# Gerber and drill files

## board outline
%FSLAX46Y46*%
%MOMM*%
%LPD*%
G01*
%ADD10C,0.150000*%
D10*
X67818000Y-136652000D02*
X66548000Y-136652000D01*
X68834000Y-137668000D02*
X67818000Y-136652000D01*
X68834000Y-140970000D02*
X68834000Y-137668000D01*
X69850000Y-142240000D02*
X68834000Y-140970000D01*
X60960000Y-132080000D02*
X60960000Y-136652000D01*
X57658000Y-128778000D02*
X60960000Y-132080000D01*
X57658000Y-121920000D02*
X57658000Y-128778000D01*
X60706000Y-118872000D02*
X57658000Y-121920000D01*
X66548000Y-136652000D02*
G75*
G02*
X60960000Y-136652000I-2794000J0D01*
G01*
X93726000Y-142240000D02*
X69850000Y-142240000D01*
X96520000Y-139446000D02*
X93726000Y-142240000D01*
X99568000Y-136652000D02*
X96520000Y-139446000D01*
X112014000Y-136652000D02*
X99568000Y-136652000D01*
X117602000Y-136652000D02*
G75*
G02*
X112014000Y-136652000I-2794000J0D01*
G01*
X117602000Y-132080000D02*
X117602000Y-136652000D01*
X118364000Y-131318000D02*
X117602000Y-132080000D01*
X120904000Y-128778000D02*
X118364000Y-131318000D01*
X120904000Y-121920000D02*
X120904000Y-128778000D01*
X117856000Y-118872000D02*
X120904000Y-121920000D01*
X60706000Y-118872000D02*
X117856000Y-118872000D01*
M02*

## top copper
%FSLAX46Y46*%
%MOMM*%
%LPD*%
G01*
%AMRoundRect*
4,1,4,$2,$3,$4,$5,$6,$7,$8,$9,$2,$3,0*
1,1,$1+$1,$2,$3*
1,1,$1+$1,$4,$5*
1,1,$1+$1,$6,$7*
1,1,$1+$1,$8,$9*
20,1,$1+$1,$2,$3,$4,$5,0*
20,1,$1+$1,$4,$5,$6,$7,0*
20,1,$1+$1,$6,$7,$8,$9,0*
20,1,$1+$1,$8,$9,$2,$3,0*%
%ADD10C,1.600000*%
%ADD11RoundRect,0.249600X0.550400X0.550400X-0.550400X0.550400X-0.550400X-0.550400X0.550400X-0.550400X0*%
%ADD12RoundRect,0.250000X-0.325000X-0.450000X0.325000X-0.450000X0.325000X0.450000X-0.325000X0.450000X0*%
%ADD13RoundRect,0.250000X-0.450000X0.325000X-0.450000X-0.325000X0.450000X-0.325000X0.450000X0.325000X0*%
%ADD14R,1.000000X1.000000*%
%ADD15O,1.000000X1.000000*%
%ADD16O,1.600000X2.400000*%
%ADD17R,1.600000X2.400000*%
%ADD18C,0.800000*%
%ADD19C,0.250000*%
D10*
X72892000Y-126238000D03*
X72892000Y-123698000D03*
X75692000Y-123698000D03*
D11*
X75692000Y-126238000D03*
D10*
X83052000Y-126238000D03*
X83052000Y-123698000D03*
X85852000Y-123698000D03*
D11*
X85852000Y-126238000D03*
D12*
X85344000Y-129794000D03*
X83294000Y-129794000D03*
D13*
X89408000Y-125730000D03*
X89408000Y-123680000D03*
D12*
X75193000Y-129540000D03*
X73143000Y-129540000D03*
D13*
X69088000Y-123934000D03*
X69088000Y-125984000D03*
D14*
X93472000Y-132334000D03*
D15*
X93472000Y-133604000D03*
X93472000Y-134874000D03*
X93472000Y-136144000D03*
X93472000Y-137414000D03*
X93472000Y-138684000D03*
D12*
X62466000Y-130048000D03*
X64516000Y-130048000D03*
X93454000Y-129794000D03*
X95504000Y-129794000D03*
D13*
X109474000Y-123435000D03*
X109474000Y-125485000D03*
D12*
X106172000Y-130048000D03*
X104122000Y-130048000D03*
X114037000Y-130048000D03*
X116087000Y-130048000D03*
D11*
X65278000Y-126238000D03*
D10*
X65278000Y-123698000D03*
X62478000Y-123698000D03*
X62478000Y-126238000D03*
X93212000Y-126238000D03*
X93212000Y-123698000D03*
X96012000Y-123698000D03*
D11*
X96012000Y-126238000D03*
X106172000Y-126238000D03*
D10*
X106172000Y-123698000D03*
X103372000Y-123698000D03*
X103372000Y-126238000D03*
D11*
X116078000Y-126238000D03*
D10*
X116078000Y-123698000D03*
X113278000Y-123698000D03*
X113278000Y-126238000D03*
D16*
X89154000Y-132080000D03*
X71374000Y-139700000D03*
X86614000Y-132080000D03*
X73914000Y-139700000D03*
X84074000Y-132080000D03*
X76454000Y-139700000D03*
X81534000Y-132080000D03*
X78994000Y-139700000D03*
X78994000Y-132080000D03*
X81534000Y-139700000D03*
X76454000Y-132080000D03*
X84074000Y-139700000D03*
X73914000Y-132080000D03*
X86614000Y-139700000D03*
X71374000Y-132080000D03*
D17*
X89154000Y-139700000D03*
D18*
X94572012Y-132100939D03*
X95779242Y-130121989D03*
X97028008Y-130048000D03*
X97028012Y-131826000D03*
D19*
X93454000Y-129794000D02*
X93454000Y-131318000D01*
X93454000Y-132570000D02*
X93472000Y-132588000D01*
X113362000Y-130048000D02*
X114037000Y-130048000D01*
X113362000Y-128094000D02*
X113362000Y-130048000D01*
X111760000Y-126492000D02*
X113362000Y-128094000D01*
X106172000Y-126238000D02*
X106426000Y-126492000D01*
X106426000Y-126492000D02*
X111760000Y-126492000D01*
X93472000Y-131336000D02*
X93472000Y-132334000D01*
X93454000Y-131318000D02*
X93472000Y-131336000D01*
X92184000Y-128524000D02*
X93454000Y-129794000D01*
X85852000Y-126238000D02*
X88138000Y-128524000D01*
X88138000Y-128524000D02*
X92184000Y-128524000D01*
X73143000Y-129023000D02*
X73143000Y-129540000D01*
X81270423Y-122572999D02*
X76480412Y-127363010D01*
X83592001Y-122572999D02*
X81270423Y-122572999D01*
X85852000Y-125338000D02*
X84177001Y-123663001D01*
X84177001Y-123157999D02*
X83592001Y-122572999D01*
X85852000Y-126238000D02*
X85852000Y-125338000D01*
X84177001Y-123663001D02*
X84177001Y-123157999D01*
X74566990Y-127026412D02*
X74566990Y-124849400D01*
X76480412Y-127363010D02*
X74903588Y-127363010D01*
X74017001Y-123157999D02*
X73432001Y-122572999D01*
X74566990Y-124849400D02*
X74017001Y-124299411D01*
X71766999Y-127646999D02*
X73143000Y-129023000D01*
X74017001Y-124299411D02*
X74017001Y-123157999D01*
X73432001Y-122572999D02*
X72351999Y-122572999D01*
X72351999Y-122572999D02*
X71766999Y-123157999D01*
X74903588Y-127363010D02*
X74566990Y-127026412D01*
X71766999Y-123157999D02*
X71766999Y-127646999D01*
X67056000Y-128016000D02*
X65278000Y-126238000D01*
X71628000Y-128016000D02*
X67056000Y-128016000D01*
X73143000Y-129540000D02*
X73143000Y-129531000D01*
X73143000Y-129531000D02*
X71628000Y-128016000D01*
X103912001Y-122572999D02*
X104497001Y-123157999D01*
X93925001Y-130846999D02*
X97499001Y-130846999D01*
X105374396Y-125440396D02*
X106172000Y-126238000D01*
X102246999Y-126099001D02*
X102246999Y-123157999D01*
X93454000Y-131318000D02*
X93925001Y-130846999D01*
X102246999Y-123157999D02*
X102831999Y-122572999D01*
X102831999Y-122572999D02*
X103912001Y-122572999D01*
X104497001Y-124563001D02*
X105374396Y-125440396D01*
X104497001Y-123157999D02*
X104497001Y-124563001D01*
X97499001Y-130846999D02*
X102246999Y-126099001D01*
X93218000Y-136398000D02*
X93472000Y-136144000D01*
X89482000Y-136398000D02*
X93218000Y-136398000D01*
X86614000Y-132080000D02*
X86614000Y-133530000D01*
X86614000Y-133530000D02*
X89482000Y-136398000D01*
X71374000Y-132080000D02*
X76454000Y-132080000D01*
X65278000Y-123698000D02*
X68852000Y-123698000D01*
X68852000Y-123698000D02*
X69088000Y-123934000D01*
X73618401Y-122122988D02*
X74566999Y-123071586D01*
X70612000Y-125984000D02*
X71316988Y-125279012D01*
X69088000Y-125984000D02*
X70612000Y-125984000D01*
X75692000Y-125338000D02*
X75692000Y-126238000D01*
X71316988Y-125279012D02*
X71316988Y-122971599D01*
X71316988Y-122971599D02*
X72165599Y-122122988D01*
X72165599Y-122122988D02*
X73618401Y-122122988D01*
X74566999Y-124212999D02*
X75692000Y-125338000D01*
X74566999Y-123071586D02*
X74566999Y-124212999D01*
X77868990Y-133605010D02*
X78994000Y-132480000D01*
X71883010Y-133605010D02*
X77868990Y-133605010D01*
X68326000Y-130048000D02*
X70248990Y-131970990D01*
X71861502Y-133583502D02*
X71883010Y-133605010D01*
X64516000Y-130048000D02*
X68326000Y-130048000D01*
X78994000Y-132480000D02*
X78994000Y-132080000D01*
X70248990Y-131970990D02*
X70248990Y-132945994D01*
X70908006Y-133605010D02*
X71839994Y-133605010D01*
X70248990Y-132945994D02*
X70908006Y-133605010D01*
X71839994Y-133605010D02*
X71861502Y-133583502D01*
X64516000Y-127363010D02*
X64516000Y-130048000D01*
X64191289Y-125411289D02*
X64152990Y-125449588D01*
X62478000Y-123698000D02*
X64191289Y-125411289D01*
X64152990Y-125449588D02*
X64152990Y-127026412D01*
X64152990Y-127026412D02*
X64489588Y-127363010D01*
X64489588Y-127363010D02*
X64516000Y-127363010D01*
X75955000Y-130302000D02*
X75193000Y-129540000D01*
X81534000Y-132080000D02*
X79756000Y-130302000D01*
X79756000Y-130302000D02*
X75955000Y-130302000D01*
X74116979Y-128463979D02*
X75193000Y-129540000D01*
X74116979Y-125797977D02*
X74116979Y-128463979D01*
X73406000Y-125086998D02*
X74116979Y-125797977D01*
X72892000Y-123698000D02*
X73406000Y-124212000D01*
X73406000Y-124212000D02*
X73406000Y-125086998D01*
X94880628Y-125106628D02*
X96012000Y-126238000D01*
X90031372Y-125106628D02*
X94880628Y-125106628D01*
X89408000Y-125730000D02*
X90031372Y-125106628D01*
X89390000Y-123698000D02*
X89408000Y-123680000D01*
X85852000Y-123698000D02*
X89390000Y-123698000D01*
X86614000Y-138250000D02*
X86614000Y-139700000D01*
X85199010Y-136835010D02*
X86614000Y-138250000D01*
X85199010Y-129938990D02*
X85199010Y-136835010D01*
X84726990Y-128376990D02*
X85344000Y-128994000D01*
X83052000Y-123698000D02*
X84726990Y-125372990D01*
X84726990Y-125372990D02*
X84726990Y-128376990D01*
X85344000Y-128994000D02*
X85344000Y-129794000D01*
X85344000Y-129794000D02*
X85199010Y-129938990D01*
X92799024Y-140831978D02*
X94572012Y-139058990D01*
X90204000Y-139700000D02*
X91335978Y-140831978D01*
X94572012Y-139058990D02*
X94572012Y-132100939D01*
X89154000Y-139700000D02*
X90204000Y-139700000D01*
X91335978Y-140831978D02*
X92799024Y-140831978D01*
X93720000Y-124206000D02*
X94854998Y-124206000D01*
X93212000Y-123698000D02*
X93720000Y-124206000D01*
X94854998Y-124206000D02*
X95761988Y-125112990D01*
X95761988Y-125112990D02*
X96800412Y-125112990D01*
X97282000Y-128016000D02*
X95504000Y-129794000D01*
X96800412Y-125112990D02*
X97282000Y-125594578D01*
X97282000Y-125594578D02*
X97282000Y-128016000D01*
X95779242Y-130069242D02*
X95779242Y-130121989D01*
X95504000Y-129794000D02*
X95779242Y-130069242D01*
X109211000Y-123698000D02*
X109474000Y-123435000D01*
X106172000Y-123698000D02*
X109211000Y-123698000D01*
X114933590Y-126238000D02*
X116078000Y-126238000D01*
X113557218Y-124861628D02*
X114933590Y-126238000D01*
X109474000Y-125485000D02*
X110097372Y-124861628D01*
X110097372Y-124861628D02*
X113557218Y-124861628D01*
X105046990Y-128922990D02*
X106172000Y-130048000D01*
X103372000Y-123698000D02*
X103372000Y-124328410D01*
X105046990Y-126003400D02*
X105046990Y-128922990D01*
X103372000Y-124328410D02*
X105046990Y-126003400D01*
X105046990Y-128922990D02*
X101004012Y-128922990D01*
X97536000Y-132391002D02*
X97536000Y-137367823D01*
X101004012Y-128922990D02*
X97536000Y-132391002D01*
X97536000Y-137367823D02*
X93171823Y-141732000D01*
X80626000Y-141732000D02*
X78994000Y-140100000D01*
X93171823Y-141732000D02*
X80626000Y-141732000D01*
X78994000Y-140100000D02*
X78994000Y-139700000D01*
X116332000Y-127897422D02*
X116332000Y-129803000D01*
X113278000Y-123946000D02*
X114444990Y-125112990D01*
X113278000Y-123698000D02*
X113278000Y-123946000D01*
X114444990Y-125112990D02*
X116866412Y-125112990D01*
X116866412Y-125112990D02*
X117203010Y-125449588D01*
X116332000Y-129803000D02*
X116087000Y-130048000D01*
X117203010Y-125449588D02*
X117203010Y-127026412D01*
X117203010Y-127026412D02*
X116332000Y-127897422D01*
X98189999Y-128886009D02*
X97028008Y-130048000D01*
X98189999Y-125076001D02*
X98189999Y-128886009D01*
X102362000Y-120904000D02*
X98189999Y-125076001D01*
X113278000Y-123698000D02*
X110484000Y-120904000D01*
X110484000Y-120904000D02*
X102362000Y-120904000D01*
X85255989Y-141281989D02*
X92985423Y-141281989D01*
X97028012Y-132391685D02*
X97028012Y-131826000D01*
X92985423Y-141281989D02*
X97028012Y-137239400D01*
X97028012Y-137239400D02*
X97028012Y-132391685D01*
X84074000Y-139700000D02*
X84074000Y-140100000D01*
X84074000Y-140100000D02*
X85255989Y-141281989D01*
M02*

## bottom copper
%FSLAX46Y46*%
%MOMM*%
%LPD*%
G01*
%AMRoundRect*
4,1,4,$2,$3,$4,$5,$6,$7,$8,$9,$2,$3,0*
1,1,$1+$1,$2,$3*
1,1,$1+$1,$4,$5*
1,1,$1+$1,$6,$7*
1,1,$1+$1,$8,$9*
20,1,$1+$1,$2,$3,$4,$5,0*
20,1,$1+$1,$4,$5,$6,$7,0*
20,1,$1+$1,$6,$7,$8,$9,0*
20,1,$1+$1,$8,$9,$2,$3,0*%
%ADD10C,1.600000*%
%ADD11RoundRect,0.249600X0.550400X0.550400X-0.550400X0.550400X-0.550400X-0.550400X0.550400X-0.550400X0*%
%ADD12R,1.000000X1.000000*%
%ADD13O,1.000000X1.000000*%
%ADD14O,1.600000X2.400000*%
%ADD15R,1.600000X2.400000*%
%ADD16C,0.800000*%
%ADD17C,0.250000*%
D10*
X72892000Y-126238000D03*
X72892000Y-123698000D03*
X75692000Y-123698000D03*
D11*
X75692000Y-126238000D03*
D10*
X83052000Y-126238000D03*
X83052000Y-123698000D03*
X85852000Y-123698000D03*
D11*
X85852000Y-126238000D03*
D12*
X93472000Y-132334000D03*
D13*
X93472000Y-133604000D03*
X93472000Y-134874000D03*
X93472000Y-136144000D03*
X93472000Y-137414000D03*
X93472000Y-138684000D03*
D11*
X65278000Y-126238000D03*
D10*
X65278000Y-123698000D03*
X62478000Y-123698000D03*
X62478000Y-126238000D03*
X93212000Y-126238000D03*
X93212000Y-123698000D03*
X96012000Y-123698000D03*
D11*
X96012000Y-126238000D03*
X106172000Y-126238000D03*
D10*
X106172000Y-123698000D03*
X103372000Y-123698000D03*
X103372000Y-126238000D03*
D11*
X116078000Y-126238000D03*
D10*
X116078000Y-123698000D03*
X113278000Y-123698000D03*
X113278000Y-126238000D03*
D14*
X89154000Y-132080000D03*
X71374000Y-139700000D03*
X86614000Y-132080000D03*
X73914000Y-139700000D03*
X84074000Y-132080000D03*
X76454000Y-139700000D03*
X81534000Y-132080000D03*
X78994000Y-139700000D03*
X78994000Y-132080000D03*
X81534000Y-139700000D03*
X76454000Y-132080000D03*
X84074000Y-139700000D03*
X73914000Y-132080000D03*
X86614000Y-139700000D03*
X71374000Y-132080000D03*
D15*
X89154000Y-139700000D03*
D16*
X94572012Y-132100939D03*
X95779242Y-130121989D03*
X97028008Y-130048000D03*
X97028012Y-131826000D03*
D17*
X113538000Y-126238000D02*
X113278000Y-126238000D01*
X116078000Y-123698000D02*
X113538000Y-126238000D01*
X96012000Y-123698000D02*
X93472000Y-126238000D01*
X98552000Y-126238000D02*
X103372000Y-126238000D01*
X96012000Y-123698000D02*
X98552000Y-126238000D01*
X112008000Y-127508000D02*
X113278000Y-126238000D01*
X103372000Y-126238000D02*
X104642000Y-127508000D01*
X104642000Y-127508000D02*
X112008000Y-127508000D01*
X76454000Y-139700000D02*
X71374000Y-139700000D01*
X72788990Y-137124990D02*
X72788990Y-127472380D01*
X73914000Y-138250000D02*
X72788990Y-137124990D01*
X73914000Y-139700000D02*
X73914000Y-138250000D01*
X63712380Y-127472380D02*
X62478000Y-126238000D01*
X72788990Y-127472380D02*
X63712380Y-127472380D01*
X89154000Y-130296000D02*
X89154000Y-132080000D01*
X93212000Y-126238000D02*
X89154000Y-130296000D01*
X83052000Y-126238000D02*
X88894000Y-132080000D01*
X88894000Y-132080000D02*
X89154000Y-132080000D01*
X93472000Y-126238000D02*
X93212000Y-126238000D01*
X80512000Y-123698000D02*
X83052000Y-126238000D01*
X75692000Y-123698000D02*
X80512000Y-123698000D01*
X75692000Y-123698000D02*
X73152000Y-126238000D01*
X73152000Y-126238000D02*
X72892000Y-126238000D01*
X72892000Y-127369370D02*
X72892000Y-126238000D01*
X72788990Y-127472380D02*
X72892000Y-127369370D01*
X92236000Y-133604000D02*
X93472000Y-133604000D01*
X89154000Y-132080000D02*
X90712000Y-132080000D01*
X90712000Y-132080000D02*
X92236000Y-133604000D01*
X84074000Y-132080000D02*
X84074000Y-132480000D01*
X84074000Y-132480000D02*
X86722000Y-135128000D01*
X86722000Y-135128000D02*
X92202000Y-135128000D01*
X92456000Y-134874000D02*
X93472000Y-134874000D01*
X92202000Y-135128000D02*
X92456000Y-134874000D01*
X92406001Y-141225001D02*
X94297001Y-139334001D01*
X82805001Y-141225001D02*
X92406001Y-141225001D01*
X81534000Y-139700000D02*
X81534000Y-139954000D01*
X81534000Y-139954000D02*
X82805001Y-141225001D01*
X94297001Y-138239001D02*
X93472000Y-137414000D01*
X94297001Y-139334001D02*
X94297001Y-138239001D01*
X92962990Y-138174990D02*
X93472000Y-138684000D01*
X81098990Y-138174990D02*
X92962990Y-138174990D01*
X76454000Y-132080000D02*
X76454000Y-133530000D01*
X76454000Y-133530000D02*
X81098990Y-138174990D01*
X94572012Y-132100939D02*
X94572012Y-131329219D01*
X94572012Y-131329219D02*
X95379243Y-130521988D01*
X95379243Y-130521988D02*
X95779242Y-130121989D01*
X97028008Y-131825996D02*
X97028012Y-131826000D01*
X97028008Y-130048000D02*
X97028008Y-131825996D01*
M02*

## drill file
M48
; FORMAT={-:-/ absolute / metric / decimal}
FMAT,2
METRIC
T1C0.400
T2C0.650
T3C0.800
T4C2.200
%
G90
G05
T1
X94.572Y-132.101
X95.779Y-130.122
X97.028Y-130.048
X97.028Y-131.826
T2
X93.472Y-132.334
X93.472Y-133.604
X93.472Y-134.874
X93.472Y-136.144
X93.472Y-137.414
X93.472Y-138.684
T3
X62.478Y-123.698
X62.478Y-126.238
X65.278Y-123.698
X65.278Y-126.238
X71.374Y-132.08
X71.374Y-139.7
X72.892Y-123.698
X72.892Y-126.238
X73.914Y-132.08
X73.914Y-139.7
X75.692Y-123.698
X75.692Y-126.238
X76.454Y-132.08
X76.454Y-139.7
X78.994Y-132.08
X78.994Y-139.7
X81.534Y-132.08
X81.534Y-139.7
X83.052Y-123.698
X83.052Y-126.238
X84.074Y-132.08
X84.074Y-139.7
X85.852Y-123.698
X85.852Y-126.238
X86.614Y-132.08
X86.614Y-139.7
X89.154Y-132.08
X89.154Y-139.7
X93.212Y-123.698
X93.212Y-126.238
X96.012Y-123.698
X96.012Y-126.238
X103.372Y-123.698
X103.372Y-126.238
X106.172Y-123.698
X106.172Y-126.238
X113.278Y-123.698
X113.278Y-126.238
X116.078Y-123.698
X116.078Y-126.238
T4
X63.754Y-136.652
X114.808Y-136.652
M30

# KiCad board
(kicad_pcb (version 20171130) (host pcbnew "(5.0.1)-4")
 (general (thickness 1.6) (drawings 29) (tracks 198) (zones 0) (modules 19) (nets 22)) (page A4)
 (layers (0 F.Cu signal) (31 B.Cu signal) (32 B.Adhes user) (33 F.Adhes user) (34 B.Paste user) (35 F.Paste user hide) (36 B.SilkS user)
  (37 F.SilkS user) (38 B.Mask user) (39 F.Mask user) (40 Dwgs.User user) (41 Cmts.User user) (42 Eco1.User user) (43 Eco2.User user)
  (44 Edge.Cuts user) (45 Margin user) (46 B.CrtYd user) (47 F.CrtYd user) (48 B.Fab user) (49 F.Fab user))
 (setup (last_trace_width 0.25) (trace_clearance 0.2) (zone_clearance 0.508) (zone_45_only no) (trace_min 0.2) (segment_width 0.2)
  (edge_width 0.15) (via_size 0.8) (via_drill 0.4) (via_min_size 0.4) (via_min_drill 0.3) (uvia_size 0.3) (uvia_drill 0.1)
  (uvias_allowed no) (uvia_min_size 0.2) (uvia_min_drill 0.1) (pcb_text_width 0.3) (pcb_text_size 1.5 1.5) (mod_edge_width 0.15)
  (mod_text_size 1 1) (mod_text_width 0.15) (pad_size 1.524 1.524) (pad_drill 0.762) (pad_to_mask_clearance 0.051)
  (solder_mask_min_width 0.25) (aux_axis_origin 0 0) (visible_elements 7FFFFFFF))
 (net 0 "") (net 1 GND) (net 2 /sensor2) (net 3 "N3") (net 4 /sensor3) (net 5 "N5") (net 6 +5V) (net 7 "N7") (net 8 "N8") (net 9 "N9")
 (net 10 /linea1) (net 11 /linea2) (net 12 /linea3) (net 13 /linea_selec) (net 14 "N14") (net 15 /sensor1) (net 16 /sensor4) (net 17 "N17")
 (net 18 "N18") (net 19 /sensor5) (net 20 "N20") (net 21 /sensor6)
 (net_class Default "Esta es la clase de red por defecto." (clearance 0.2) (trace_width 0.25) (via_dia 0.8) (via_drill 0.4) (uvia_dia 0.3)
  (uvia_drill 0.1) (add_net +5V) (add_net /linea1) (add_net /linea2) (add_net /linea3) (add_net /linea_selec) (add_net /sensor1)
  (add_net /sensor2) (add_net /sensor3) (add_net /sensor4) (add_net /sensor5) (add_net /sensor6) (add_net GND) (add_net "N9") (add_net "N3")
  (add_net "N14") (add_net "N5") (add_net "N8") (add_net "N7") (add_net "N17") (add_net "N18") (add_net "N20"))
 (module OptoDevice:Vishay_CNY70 (layer F.Cu) (at 75.692 126.238 180)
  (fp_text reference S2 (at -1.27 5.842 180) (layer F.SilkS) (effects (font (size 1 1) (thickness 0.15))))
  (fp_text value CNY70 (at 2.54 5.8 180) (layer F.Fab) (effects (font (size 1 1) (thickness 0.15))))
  (pad 4 thru_hole circle (at 2.8 0 180) (size 1.6 1.6) (drill 0.8) (layers *.Cu *.Mask) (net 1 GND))
  (pad 3 thru_hole circle (at 2.8 2.54 180) (size 1.6 1.6) (drill 0.8) (layers *.Cu *.Mask) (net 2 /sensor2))
  (pad 2 thru_hole circle (at 0 2.54 180) (size 1.6 1.6) (drill 0.8) (layers *.Cu *.Mask) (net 1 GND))
  (pad 1 thru_hole roundrect (at 0 0 180) (size 1.6 1.6) (drill 0.8) (layers *.Cu *.Mask) (roundrect_rratio 0.156) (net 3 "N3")))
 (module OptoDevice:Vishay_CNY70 (layer F.Cu) (at 85.852 126.238 180)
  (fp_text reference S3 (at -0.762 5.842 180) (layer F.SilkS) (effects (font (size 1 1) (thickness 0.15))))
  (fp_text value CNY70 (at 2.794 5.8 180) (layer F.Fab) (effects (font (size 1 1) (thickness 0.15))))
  (pad 4 thru_hole circle (at 2.8 0 180) (size 1.6 1.6) (drill 0.8) (layers *.Cu *.Mask) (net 1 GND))
  (pad 3 thru_hole circle (at 2.8 2.54 180) (size 1.6 1.6) (drill 0.8) (layers *.Cu *.Mask) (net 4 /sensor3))
  (pad 2 thru_hole circle (at 0 2.54 180) (size 1.6 1.6) (drill 0.8) (layers *.Cu *.Mask) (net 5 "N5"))
  (pad 1 thru_hole roundrect (at 0 0 180) (size 1.6 1.6) (drill 0.8) (layers *.Cu *.Mask) (roundrect_rratio 0.156) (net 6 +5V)))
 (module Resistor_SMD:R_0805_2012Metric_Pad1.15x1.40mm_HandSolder (layer F.Cu) (at 84.319 129.794)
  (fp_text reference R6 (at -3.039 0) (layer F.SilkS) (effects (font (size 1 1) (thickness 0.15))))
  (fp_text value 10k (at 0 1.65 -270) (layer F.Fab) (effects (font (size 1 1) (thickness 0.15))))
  (pad 2 smd roundrect (at 1.025 0) (size 1.15 1.4) (layers F.Cu F.Paste F.Mask) (roundrect_rratio 0.217391) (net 4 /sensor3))
  (pad 1 smd roundrect (at -1.025 0) (size 1.15 1.4) (layers F.Cu F.Paste F.Mask) (roundrect_rratio 0.217391) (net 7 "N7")))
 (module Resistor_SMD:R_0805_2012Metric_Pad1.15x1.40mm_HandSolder (layer F.Cu) (at 89.408 124.705 270)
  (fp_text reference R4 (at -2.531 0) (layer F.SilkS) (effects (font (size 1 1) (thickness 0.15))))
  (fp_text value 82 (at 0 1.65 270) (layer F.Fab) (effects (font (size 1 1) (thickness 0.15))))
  (pad 2 smd roundrect (at 1.025 0 270) (size 1.15 1.4) (layers F.Cu F.Paste F.Mask) (roundrect_rratio 0.217391) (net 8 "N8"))
  (pad 1 smd roundrect (at -1.025 0 270) (size 1.15 1.4) (layers F.Cu F.Paste F.Mask) (roundrect_rratio 0.217391) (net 5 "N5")))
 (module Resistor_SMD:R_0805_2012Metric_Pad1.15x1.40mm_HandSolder (layer F.Cu) (at 74.168 129.54)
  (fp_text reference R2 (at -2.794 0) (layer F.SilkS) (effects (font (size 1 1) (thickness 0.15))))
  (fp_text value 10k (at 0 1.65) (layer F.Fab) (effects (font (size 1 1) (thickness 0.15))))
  (pad 2 smd roundrect (at 1.025 0) (size 1.15 1.4) (layers F.Cu F.Paste F.Mask) (roundrect_rratio 0.217391) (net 2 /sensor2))
  (pad 1 smd roundrect (at -1.025 0) (size 1.15 1.4) (layers F.Cu F.Paste F.Mask) (roundrect_rratio 0.217391) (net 6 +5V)))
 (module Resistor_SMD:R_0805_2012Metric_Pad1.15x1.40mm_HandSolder (layer F.Cu) (at 69.088 124.959 270)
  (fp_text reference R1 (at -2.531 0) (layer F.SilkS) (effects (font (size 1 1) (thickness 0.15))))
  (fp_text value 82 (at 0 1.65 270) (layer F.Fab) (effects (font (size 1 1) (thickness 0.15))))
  (pad 1 smd roundrect (at -1.025 0 270) (size 1.15 1.4) (layers F.Cu F.Paste F.Mask) (roundrect_rratio 0.217391) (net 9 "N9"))
  (pad 2 smd roundrect (at 1.025 0 270) (size 1.15 1.4) (layers F.Cu F.Paste F.Mask) (roundrect_rratio 0.217391) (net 3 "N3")))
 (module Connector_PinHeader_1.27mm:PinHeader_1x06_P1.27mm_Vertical (layer B.Cu) (at 93.472 132.334 180)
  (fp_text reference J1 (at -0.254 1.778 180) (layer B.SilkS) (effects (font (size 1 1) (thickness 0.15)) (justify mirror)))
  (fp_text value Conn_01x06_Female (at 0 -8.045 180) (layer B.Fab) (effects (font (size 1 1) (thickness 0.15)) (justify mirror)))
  (pad 1 thru_hole rect (at 0 0 180) (size 1 1) (drill 0.65) (layers *.Cu *.Mask) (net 6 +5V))
  (pad 2 thru_hole oval (at 0 -1.27 180) (size 1 1) (drill 0.65) (layers *.Cu *.Mask) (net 1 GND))
  (pad 3 thru_hole oval (at 0 -2.54 180) (size 1 1) (drill 0.65) (layers *.Cu *.Mask) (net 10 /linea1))
  (pad 4 thru_hole oval (at 0 -3.81 180) (size 1 1) (drill 0.65) (layers *.Cu *.Mask) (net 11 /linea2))
  (pad 5 thru_hole oval (at 0 -5.08 180) (size 1 1) (drill 0.65) (layers *.Cu *.Mask) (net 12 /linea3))
  (pad 6 thru_hole oval (at 0 -6.35 180) (size 1 1) (drill 0.65) (layers *.Cu *.Mask) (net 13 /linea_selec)))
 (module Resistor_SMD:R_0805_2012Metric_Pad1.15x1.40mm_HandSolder (layer F.Cu) (at 63.491 130.048)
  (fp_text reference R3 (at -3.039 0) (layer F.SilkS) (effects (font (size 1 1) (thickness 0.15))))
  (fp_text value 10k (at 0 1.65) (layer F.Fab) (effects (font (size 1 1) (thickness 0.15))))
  (pad 1 smd roundrect (at -1.025 0) (size 1.15 1.4) (layers F.Cu F.Paste F.Mask) (roundrect_rratio 0.217391) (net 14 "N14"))
  (pad 2 smd roundrect (at 1.025 0) (size 1.15 1.4) (layers F.Cu F.Paste F.Mask) (roundrect_rratio 0.217391) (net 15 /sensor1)))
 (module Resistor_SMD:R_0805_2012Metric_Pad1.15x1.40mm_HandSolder (layer F.Cu) (at 94.479 129.794)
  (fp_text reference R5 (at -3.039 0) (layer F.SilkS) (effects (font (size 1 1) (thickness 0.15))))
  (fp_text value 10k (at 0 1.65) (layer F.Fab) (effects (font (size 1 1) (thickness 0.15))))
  (pad 1 smd roundrect (at -1.025 0) (size 1.15 1.4) (layers F.Cu F.Paste F.Mask) (roundrect_rratio 0.217391) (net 6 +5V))
  (pad 2 smd roundrect (at 1.025 0) (size 1.15 1.4) (layers F.Cu F.Paste F.Mask) (roundrect_rratio 0.217391) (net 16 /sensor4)))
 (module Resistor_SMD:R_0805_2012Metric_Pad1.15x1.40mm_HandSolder (layer F.Cu) (at 109.474 124.46 270)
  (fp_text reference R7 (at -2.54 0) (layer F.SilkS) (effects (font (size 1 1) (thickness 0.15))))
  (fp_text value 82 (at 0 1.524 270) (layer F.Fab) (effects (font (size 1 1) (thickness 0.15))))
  (pad 1 smd roundrect (at -1.025 0 270) (size 1.15 1.4) (layers F.Cu F.Paste F.Mask) (roundrect_rratio 0.217391) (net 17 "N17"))
  (pad 2 smd roundrect (at 1.025 0 270) (size 1.15 1.4) (layers F.Cu F.Paste F.Mask) (roundrect_rratio 0.217391) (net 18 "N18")))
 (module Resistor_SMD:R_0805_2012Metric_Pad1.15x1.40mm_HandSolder (layer F.Cu) (at 105.147 130.048)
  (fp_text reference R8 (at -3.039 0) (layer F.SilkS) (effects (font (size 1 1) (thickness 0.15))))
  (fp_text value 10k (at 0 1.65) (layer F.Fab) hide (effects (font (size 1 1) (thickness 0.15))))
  (pad 2 smd roundrect (at 1.025 0) (size 1.15 1.4) (layers F.Cu F.Paste F.Mask) (roundrect_rratio 0.217391) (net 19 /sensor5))
  (pad 1 smd roundrect (at -1.025 0) (size 1.15 1.4) (layers F.Cu F.Paste F.Mask) (roundrect_rratio 0.217391) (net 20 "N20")))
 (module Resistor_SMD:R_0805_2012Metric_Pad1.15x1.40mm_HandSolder (layer F.Cu) (at 115.062 130.048)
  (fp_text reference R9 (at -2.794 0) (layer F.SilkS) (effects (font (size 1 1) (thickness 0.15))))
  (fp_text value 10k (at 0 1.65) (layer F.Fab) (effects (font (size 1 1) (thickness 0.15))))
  (pad 1 smd roundrect (at -1.025 0) (size 1.15 1.4) (layers F.Cu F.Paste F.Mask) (roundrect_rratio 0.217391) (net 6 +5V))
  (pad 2 smd roundrect (at 1.025 0) (size 1.15 1.4) (layers F.Cu F.Paste F.Mask) (roundrect_rratio 0.217391) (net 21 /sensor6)))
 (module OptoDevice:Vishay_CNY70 (layer F.Cu) (at 65.278 126.238 180)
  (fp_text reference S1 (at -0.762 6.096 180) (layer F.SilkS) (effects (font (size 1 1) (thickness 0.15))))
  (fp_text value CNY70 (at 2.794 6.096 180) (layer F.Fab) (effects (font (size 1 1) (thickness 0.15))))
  (pad 1 thru_hole roundrect (at 0 0 180) (size 1.6 1.6) (drill 0.8) (layers *.Cu *.Mask) (roundrect_rratio 0.156) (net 6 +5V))
  (pad 2 thru_hole circle (at 0 2.54 180) (size 1.6 1.6) (drill 0.8) (layers *.Cu *.Mask) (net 9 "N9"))
  (pad 3 thru_hole circle (at 2.8 2.54 180) (size 1.6 1.6) (drill 0.8) (layers *.Cu *.Mask) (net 15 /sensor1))
  (pad 4 thru_hole circle (at 2.8 0 180) (size 1.6 1.6) (drill 0.8) (layers *.Cu *.Mask) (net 1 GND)))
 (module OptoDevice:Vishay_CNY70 (layer F.Cu) (at 96.012 126.238 180)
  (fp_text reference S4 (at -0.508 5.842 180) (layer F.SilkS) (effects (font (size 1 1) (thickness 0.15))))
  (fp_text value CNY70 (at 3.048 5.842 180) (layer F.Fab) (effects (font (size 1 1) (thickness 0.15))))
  (pad 4 thru_hole circle (at 2.8 0 180) (size 1.6 1.6) (drill 0.8) (layers *.Cu *.Mask) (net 1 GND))
  (pad 3 thru_hole circle (at 2.8 2.54 180) (size 1.6 1.6) (drill 0.8) (layers *.Cu *.Mask) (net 16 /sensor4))
  (pad 2 thru_hole circle (at 0 2.54 180) (size 1.6 1.6) (drill 0.8) (layers *.Cu *.Mask) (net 1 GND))
  (pad 1 thru_hole roundrect (at 0 0 180) (size 1.6 1.6) (drill 0.8) (layers *.Cu *.Mask) (roundrect_rratio 0.156) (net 8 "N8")))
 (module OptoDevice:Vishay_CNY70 (layer F.Cu) (at 106.172 126.238 180)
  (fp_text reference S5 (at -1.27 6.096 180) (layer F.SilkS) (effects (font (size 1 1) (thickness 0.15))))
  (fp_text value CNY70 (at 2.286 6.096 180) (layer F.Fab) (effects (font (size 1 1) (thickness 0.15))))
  (pad 1 thru_hole roundrect (at 0 0 180) (size 1.6 1.6) (drill 0.8) (layers *.Cu *.Mask) (roundrect_rratio 0.156) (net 6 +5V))
  (pad 2 thru_hole circle (at 0 2.54 180) (size 1.6 1.6) (drill 0.8) (layers *.Cu *.Mask) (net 17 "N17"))
  (pad 3 thru_hole circle (at 2.8 2.54 180) (size 1.6 1.6) (drill 0.8) (layers *.Cu *.Mask) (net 19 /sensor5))
  (pad 4 thru_hole circle (at 2.8 0 180) (size 1.6 1.6) (drill 0.8) (layers *.Cu *.Mask) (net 1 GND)))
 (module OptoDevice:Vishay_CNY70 (layer F.Cu) (at 116.078 126.238 180)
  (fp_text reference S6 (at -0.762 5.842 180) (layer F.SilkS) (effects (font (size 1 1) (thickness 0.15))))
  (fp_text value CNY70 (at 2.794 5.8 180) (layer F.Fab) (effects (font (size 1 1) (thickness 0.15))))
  (pad 1 thru_hole roundrect (at 0 0 180) (size 1.6 1.6) (drill 0.8) (layers *.Cu *.Mask) (roundrect_rratio 0.156) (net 18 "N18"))
  (pad 2 thru_hole circle (at 0 2.54 180) (size 1.6 1.6) (drill 0.8) (layers *.Cu *.Mask) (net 1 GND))
  (pad 3 thru_hole circle (at 2.8 2.54 180) (size 1.6 1.6) (drill 0.8) (layers *.Cu *.Mask) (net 21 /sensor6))
  (pad 4 thru_hole circle (at 2.8 0 180) (size 1.6 1.6) (drill 0.8) (layers *.Cu *.Mask) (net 1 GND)))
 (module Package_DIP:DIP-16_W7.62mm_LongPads (layer B.Cu) (at 89.154 139.7 90)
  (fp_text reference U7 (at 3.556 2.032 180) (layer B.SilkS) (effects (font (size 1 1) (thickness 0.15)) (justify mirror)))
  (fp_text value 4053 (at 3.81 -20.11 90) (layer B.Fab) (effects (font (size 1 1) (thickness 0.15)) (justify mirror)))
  (pad 16 thru_hole oval (at 7.62 0 90) (size 2.4 1.6) (drill 0.8) (layers *.Cu *.Mask) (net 1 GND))
  (pad 8 thru_hole oval (at 0 -17.78 90) (size 2.4 1.6) (drill 0.8) (layers *.Cu *.Mask) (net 1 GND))
  (pad 15 thru_hole oval (at 7.62 -2.54 90) (size 2.4 1.6) (drill 0.8) (layers *.Cu *.Mask) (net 11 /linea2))
  (pad 7 thru_hole oval (at 0 -15.24 90) (size 2.4 1.6) (drill 0.8) (layers *.Cu *.Mask) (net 1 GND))
  (pad 14 thru_hole oval (at 7.62 -5.08 90) (size 2.4 1.6) (drill 0.8) (layers *.Cu *.Mask) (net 10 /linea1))
  (pad 6 thru_hole oval (at 0 -12.7 90) (size 2.4 1.6) (drill 0.8) (layers *.Cu *.Mask) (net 1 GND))
  (pad 13 thru_hole oval (at 7.62 -7.62 90) (size 2.4 1.6) (drill 0.8) (layers *.Cu *.Mask) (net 2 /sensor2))
  (pad 5 thru_hole oval (at 0 -10.16 90) (size 2.4 1.6) (drill 0.8) (layers *.Cu *.Mask) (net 19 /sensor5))
  (pad 12 thru_hole oval (at 7.62 -10.16 90) (size 2.4 1.6) (drill 0.8) (layers *.Cu *.Mask) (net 15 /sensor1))
  (pad 4 thru_hole oval (at 0 -7.62 90) (size 2.4 1.6) (drill 0.8) (layers *.Cu *.Mask) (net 12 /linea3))
  (pad 11 thru_hole oval (at 7.62 -12.7 90) (size 2.4 1.6) (drill 0.8) (layers *.Cu *.Mask) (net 13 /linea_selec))
  (pad 3 thru_hole oval (at 0 -5.08 90) (size 2.4 1.6) (drill 0.8) (layers *.Cu *.Mask) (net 21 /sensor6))
  (pad 10 thru_hole oval (at 7.62 -15.24 90) (size 2.4 1.6) (drill 0.8) (layers *.Cu *.Mask) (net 13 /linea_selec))
  (pad 2 thru_hole oval (at 0 -2.54 90) (size 2.4 1.6) (drill 0.8) (layers *.Cu *.Mask) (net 4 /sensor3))
  (pad 9 thru_hole oval (at 7.62 -17.78 90) (size 2.4 1.6) (drill 0.8) (layers *.Cu *.Mask) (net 13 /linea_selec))
  (pad 1 thru_hole rect (at 0 0 90) (size 2.4 1.6) (drill 0.8) (layers *.Cu *.Mask) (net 16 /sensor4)))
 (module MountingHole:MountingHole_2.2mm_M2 (layer F.Cu) (at 114.808 136.652)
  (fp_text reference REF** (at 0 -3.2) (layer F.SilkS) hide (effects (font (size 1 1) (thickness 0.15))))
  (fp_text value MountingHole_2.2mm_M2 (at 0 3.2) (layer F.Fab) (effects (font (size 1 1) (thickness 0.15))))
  (pad 1 np_thru_hole circle (at 0 0) (size 2.2 2.2) (drill 2.2) (layers *.Cu *.Mask)))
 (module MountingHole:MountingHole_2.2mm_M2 (layer F.Cu) (at 63.754 136.652)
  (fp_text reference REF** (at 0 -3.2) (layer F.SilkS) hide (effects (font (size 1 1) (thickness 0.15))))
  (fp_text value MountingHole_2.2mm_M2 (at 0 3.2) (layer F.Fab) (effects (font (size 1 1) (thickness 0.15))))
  (pad 1 np_thru_hole circle (at 0 0) (size 2.2 2.2) (drill 2.2) (layers *.Cu *.Mask)))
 (gr_line (start 67.818 136.652) (end 66.548 136.652) (layer Edge.Cuts) (width 0.15))
 (gr_line (start 68.834 137.668) (end 67.818 136.652) (layer Edge.Cuts) (width 0.15))
 (gr_line (start 68.834 140.97) (end 68.834 137.668) (layer Edge.Cuts) (width 0.15))
 (gr_line (start 69.85 142.24) (end 68.834 140.97) (layer Edge.Cuts) (width 0.15))
 (gr_line (start 60.96 132.08) (end 60.96 136.652) (layer Edge.Cuts) (width 0.15))
 (gr_line (start 57.658 128.778) (end 60.96 132.08) (layer Edge.Cuts) (width 0.15))
 (gr_line (start 57.658 121.92) (end 57.658 128.778) (layer Edge.Cuts) (width 0.15))
 (gr_line (start 60.706 118.872) (end 57.658 121.92) (layer Edge.Cuts) (width 0.15))
 (gr_arc (start 63.754 136.652) (end 60.96 136.652) (angle -180) (layer Edge.Cuts) (width 0.15))
 (gr_line (start 93.726 142.24) (end 69.85 142.24) (layer Edge.Cuts) (width 0.15))
 (gr_line (start 96.52 139.446) (end 93.726 142.24) (layer Edge.Cuts) (width 0.15))
 (gr_line (start 99.568 136.652) (end 96.52 139.446) (layer Edge.Cuts) (width 0.15))
 (gr_line (start 112.014 136.652) (end 99.568 136.652) (layer Edge.Cuts) (width 0.15))
 (gr_arc (start 114.808 136.652) (end 112.014 136.652) (angle -180) (layer Edge.Cuts) (width 0.15))
 (gr_line (start 117.602 132.08) (end 117.602 136.652) (layer Edge.Cuts) (width 0.15))
 (gr_line (start 118.364 131.318) (end 117.602 132.08) (layer Edge.Cuts) (width 0.15))
 (gr_line (start 120.904 128.778) (end 118.364 131.318) (layer Edge.Cuts) (width 0.15))
 (gr_line (start 120.904 121.92) (end 120.904 128.778) (layer Edge.Cuts) (width 0.15))
 (gr_line (start 117.856 118.872) (end 120.904 121.92) (layer Edge.Cuts) (width 0.15))
 (gr_line (start 60.706 118.872) (end 117.856 118.872) (layer Edge.Cuts) (width 0.15))
 (segment (start 93.454 129.794) (end 93.454 131.318) (width 0.25) (layer F.Cu) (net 6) (status 10))
 (segment (start 93.454 132.57) (end 93.472 132.588) (width 0.25) (layer F.Cu) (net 6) (status 30))
 (segment (start 113.362 130.048) (end 114.037 130.048) (width 0.25) (layer F.Cu) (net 6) (status 20))
 (segment (start 113.362 128.094) (end 113.362 130.048) (width 0.25) (layer F.Cu) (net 6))
 (segment (start 111.76 126.492) (end 113.362 128.094) (width 0.25) (layer F.Cu) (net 6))
 (segment (start 106.172 126.238) (end 106.426 126.492) (width 0.25) (layer F.Cu) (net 6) (status 30))
 (segment (start 106.426 126.492) (end 111.76 126.492) (width 0.25) (layer F.Cu) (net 6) (status 10))
 (segment (start 93.472 131.336) (end 93.472 132.334) (width 0.25) (layer F.Cu) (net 6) (status 20))
 (segment (start 93.454 131.318) (end 93.472 131.336) (width 0.25) (layer F.Cu) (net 6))
 (segment (start 92.184 128.524) (end 93.454 129.794) (width 0.25) (layer F.Cu) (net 6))
 (segment (start 85.852 126.238) (end 88.138 128.524) (width 0.25) (layer F.Cu) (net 6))
 (segment (start 88.138 128.524) (end 92.184 128.524) (width 0.25) (layer F.Cu) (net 6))
 (segment (start 73.143 129.023) (end 73.143 129.54) (width 0.25) (layer F.Cu) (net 6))
 (segment (start 81.270423 122.572999) (end 76.480412 127.36301) (width 0.25) (layer F.Cu) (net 6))
 (segment (start 83.592001 122.572999) (end 81.270423 122.572999) (width 0.25) (layer F.Cu) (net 6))
 (segment (start 85.852 125.338) (end 84.177001 123.663001) (width 0.25) (layer F.Cu) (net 6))
 (segment (start 84.177001 123.157999) (end 83.592001 122.572999) (width 0.25) (layer F.Cu) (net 6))
 (segment (start 85.852 126.238) (end 85.852 125.338) (width 0.25) (layer F.Cu) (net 6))
 (segment (start 84.177001 123.663001) (end 84.177001 123.157999) (width 0.25) (layer F.Cu) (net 6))
 (segment (start 74.56699 127.026412) (end 74.56699 124.8494) (width 0.25) (layer F.Cu) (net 6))
 (segment (start 76.480412 127.36301) (end 74.903588 127.36301) (width 0.25) (layer F.Cu) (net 6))
 (segment (start 74.017001 123.157999) (end 73.432001 122.572999) (width 0.25) (layer F.Cu) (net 6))
 (segment (start 74.56699 124.8494) (end 74.017001 124.299411) (width 0.25) (layer F.Cu) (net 6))
 (segment (start 71.766999 127.646999) (end 73.143 129.023) (width 0.25) (layer F.Cu) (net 6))
 (segment (start 74.017001 124.299411) (end 74.017001 123.157999) (width 0.25) (layer F.Cu) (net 6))
 (segment (start 73.432001 122.572999) (end 72.351999 122.572999) (width 0.25) (layer F.Cu) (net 6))
 (segment (start 72.351999 122.572999) (end 71.766999 123.157999) (width 0.25) (layer F.Cu) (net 6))
 (segment (start 74.903588 127.36301) (end 74.56699 127.026412) (width 0.25) (layer F.Cu) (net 6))
 (segment (start 71.766999 123.157999) (end 71.766999 127.646999) (width 0.25) (layer F.Cu) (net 6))
 (segment (start 67.056 128.016) (end 65.278 126.238) (width 0.25) (layer F.Cu) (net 6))
 (segment (start 71.628 128.016) (end 67.056 128.016) (width 0.25) (layer F.Cu) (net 6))
 (segment (start 73.143 129.54) (end 73.143 129.531) (width 0.25) (layer F.Cu) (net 6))
 (segment (start 73.143 129.531) (end 71.628 128.016) (width 0.25) (layer F.Cu) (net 6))
 (segment (start 103.912001 122.572999) (end 104.497001 123.157999) (width 0.25) (layer F.Cu) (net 6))
 (segment (start 93.925001 130.846999) (end 97.499001 130.846999) (width 0.25) (layer F.Cu) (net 6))
 (segment (start 105.374396 125.440396) (end 106.172 126.238) (width 0.25) (layer F.Cu) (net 6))
 (segment (start 102.246999 126.099001) (end 102.246999 123.157999) (width 0.25) (layer F.Cu) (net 6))
 (segment (start 93.454 131.318) (end 93.925001 130.846999) (width 0.25) (layer F.Cu) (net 6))
 (segment (start 102.246999 123.157999) (end 102.831999 122.572999) (width 0.25) (layer F.Cu) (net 6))
 (segment (start 102.831999 122.572999) (end 103.912001 122.572999) (width 0.25) (layer F.Cu) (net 6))
 (segment (start 104.497001 124.563001) (end 105.374396 125.440396) (width 0.25) (layer F.Cu) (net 6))
 (segment (start 104.497001 123.157999) (end 104.497001 124.563001) (width 0.25) (layer F.Cu) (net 6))
 (segment (start 97.499001 130.846999) (end 102.246999 126.099001) (width 0.25) (layer F.Cu) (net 6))
 (segment (start 113.538 126.238) (end 113.278 126.238) (width 0.25) (layer B.Cu) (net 1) (status 30))
 (segment (start 116.078 123.698) (end 113.538 126.238) (width 0.25) (layer B.Cu) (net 1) (status 30))
 (segment (start 96.012 123.698) (end 93.472 126.238) (width 0.25) (layer B.Cu) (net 1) (status 30))
 (segment (start 98.552 126.238) (end 103.372 126.238) (width 0.25) (layer B.Cu) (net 1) (status 20))
 (segment (start 96.012 123.698) (end 98.552 126.238) (width 0.25) (layer B.Cu) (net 1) (status 10))
 (segment (start 112.008 127.508) (end 113.278 126.238) (width 0.25) (layer B.Cu) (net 1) (status 20))
 (segment (start 103.372 126.238) (end 104.642 127.508) (width 0.25) (layer B.Cu) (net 1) (status 10))
 (segment (start 104.642 127.508) (end 112.008 127.508) (width 0.25) (layer B.Cu) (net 1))
 (segment (start 76.454 139.7) (end 71.374 139.7) (width 0.25) (layer B.Cu) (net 1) (status 30))
 (segment (start 72.78899 137.12499) (end 72.78899 127.47238) (width 0.25) (layer B.Cu) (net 1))
 (segment (start 73.914 138.25) (end 72.78899 137.12499) (width 0.25) (layer B.Cu) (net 1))
 (segment (start 73.914 139.7) (end 73.914 138.25) (width 0.25) (layer B.Cu) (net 1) (status 10))
 (segment (start 63.71238 127.47238) (end 62.478 126.238) (width 0.25) (layer B.Cu) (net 1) (status 20))
 (segment (start 72.78899 127.47238) (end 63.71238 127.47238) (width 0.25) (layer B.Cu) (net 1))
 (segment (start 89.154 130.296) (end 89.154 132.08) (width 0.25) (layer B.Cu) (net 1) (status 20))
 (segment (start 93.212 126.238) (end 89.154 130.296) (width 0.25) (layer B.Cu) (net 1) (status 10))
 (segment (start 83.052 126.238) (end 88.894 132.08) (width 0.25) (layer B.Cu) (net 1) (status 30))
 (segment (start 88.894 132.08) (end 89.154 132.08) (width 0.25) (layer B.Cu) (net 1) (status 30))
 (segment (start 93.472 126.238) (end 93.212 126.238) (width 0.25) (layer B.Cu) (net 1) (status 30))
 (segment (start 80.512 123.698) (end 83.052 126.238) (width 0.25) (layer B.Cu) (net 1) (status 20))
 (segment (start 75.692 123.698) (end 80.512 123.698) (width 0.25) (layer B.Cu) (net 1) (status 10))
 (segment (start 75.692 123.698) (end 73.152 126.238) (width 0.25) (layer B.Cu) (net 1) (status 30))
 (segment (start 73.152 126.238) (end 72.892 126.238) (width 0.25) (layer B.Cu) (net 1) (status 30))
 (segment (start 72.892 127.36937) (end 72.892 126.238) (width 0.25) (layer B.Cu) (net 1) (status 20))
 (segment (start 72.78899 127.47238) (end 72.892 127.36937) (width 0.25) (layer B.Cu) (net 1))
 (segment (start 92.236 133.604) (end 93.472 133.604) (width 0.25) (layer B.Cu) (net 1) (status 20))
 (segment (start 89.154 132.08) (end 90.712 132.08) (width 0.25) (layer B.Cu) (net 1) (status 10))
 (segment (start 90.712 132.08) (end 92.236 133.604) (width 0.25) (layer B.Cu) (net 1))
 (segment (start 84.074 132.08) (end 84.074 132.48) (width 0.25) (layer B.Cu) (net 10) (status 30))
 (segment (start 84.074 132.48) (end 86.722 135.128) (width 0.25) (layer B.Cu) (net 10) (status 10))
 (segment (start 86.722 135.128) (end 92.202 135.128) (width 0.25) (layer B.Cu) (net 10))
 (segment (start 92.456 134.874) (end 93.472 134.874) (width 0.25) (layer B.Cu) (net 10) (status 20))
 (segment (start 92.202 135.128) (end 92.456 134.874) (width 0.25) (layer B.Cu) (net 10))
 (segment (start 93.218 136.398) (end 93.472 136.144) (width 0.25) (layer F.Cu) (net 11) (status 30))
 (segment (start 89.482 136.398) (end 93.218 136.398) (width 0.25) (layer F.Cu) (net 11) (status 20))
 (segment (start 86.614 132.08) (end 86.614 133.53) (width 0.25) (layer F.Cu) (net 11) (status 10))
 (segment (start 86.614 133.53) (end 89.482 136.398) (width 0.25) (layer F.Cu) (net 11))
 (segment (start 92.406001 141.225001) (end 94.297001 139.334001) (width 0.25) (layer B.Cu) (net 12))
 (segment (start 82.805001 141.225001) (end 92.406001 141.225001) (width 0.25) (layer B.Cu) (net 12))
 (segment (start 81.534 139.7) (end 81.534 139.954) (width 0.25) (layer B.Cu) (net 12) (status 30))
 (segment (start 81.534 139.954) (end 82.805001 141.225001) (width 0.25) (layer B.Cu) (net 12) (status 10))
 (segment (start 94.297001 138.239001) (end 93.472 137.414) (width 0.25) (layer B.Cu) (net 12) (status 20))
 (segment (start 94.297001 139.334001) (end 94.297001 138.239001) (width 0.25) (layer B.Cu) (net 12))
 (segment (start 71.374 132.08) (end 76.454 132.08) (width 0.25) (layer F.Cu) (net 13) (status 30))
 (segment (start 92.96299 138.17499) (end 93.472 138.684) (width 0.25) (layer B.Cu) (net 13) (status 20))
 (segment (start 81.09899 138.17499) (end 92.96299 138.17499) (width 0.25) (layer B.Cu) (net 13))
 (segment (start 76.454 132.08) (end 76.454 133.53) (width 0.25) (layer B.Cu) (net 13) (status 10))
 (segment (start 76.454 133.53) (end 81.09899 138.17499) (width 0.25) (layer B.Cu) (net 13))
 (segment (start 65.278 123.698) (end 68.852 123.698) (width 0.25) (layer F.Cu) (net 9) (status 30))
 (segment (start 68.852 123.698) (end 69.088 123.934) (width 0.25) (layer F.Cu) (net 9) (status 30))
 (segment (start 73.618401 122.122988) (end 74.566999 123.071586) (width 0.25) (layer F.Cu) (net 3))
 (segment (start 70.612 125.984) (end 71.316988 125.279012) (width 0.25) (layer F.Cu) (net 3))
 (segment (start 69.088 125.984) (end 70.612 125.984) (width 0.25) (layer F.Cu) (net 3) (status 10))
 (segment (start 75.692 125.338) (end 75.692 126.238) (width 0.25) (layer F.Cu) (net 3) (status 20))
 (segment (start 71.316988 125.279012) (end 71.316988 122.971599) (width 0.25) (layer F.Cu) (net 3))
 (segment (start 71.316988 122.971599) (end 72.165599 122.122988) (width 0.25) (layer F.Cu) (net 3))
 (segment (start 72.165599 122.122988) (end 73.618401 122.122988) (width 0.25) (layer F.Cu) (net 3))
 (segment (start 74.566999 124.212999) (end 75.692 125.338) (width 0.25) (layer F.Cu) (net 3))
 (segment (start 74.566999 123.071586) (end 74.566999 124.212999) (width 0.25) (layer F.Cu) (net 3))
 (segment (start 77.86899 133.60501) (end 78.994 132.48) (width 0.25) (layer F.Cu) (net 15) (status 20))
 (segment (start 71.88301 133.60501) (end 77.86899 133.60501) (width 0.25) (layer F.Cu) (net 15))
 (segment (start 68.326 130.048) (end 70.24899 131.97099) (width 0.25) (layer F.Cu) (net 15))
 (segment (start 71.861502 133.583502) (end 71.88301 133.60501) (width 0.25) (layer F.Cu) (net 15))
 (segment (start 64.516 130.048) (end 68.326 130.048) (width 0.25) (layer F.Cu) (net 15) (status 10))
 (segment (start 78.994 132.48) (end 78.994 132.08) (width 0.25) (layer F.Cu) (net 15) (status 30))
 (segment (start 70.24899 131.97099) (end 70.24899 132.945994) (width 0.25) (layer F.Cu) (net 15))
 (segment (start 70.908006 133.60501) (end 71.839994 133.60501) (width 0.25) (layer F.Cu) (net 15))
 (segment (start 70.24899 132.945994) (end 70.908006 133.60501) (width 0.25) (layer F.Cu) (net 15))
 (segment (start 71.839994 133.60501) (end 71.861502 133.583502) (width 0.25) (layer F.Cu) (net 15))
 (segment (start 64.516 127.36301) (end 64.516 130.048) (width 0.25) (layer F.Cu) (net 15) (status 20))
 (segment (start 64.191289 125.411289) (end 64.15299 125.449588) (width 0.25) (layer F.Cu) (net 15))
 (segment (start 62.478 123.698) (end 64.191289 125.411289) (width 0.25) (layer F.Cu) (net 15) (status 10))
 (segment (start 64.15299 125.449588) (end 64.15299 127.026412) (width 0.25) (layer F.Cu) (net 15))
 (segment (start 64.15299 127.026412) (end 64.489588 127.36301) (width 0.25) (layer F.Cu) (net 15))
 (segment (start 64.489588 127.36301) (end 64.516 127.36301) (width 0.25) (layer F.Cu) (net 15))
 (segment (start 75.955 130.302) (end 75.193 129.54) (width 0.25) (layer F.Cu) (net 2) (status 20))
 (segment (start 81.534 132.08) (end 79.756 130.302) (width 0.25) (layer F.Cu) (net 2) (status 10))
 (segment (start 79.756 130.302) (end 75.955 130.302) (width 0.25) (layer F.Cu) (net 2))
 (segment (start 74.116979 128.463979) (end 75.193 129.54) (width 0.25) (layer F.Cu) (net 2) (status 20))
 (segment (start 74.116979 125.797977) (end 74.116979 128.463979) (width 0.25) (layer F.Cu) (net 2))
 (segment (start 73.406 125.086998) (end 74.116979 125.797977) (width 0.25) (layer F.Cu) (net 2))
 (segment (start 72.892 123.698) (end 73.406 124.212) (width 0.25) (layer F.Cu) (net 2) (status 30))
 (segment (start 73.406 124.212) (end 73.406 125.086998) (width 0.25) (layer F.Cu) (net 2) (status 10))
 (segment (start 94.880628 125.106628) (end 96.012 126.238) (width 0.25) (layer F.Cu) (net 8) (status 20))
 (segment (start 90.031372 125.106628) (end 94.880628 125.106628) (width 0.25) (layer F.Cu) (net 8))
 (segment (start 89.408 125.73) (end 90.031372 125.106628) (width 0.25) (layer F.Cu) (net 8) (status 10))
 (segment (start 89.39 123.698) (end 89.408 123.68) (width 0.25) (layer F.Cu) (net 5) (status 30))
 (segment (start 85.852 123.698) (end 89.39 123.698) (width 0.25) (layer F.Cu) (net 5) (status 30))
 (segment (start 86.614 138.25) (end 86.614 139.7) (width 0.25) (layer F.Cu) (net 4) (status 20))
 (segment (start 85.19901 136.83501) (end 86.614 138.25) (width 0.25) (layer F.Cu) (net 4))
 (segment (start 85.19901 129.93899) (end 85.19901 136.83501) (width 0.25) (layer F.Cu) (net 4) (status 10))
 (segment (start 84.72699 128.37699) (end 85.344 128.994) (width 0.25) (layer F.Cu) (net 4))
 (segment (start 83.052 123.698) (end 84.72699 125.37299) (width 0.25) (layer F.Cu) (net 4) (status 10))
 (segment (start 84.72699 125.37299) (end 84.72699 128.37699) (width 0.25) (layer F.Cu) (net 4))
 (segment (start 85.344 128.994) (end 85.344 129.794) (width 0.25) (layer F.Cu) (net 4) (status 20))
 (segment (start 85.344 129.794) (end 85.19901 129.93899) (width 0.25) (layer F.Cu) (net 4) (status 30))
 (segment (start 92.799024 140.831978) (end 94.572012 139.05899) (width 0.25) (layer F.Cu) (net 16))
 (via (at 94.572012 132.100939) (size 0.8) (drill 0.4) (layers F.Cu B.Cu) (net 16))
 (segment (start 90.204 139.7) (end 91.335978 140.831978) (width 0.25) (layer F.Cu) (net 16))
 (segment (start 94.572012 139.05899) (end 94.572012 132.100939) (width 0.25) (layer F.Cu) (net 16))
 (segment (start 89.154 139.7) (end 90.204 139.7) (width 0.25) (layer F.Cu) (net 16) (status 10))
 (segment (start 91.335978 140.831978) (end 92.799024 140.831978) (width 0.25) (layer F.Cu) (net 16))
 (segment (start 93.72 124.206) (end 94.854998 124.206) (width 0.25) (layer F.Cu) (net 16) (status 10))
 (segment (start 93.212 123.698) (end 93.72 124.206) (width 0.25) (layer F.Cu) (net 16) (status 30))
 (segment (start 94.854998 124.206) (end 95.761988 125.11299) (width 0.25) (layer F.Cu) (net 16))
 (segment (start 95.761988 125.11299) (end 96.800412 125.11299) (width 0.25) (layer F.Cu) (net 16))
 (segment (start 97.282 128.016) (end 95.504 129.794) (width 0.25) (layer F.Cu) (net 16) (status 20))
 (segment (start 96.800412 125.11299) (end 97.282 125.594578) (width 0.25) (layer F.Cu) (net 16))
 (segment (start 97.282 125.594578) (end 97.282 128.016) (width 0.25) (layer F.Cu) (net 16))
 (segment (start 94.572012 132.100939) (end 94.572012 131.329219) (width 0.25) (layer B.Cu) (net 16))
 (segment (start 94.572012 131.329219) (end 95.379243 130.521988) (width 0.25) (layer B.Cu) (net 16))
 (segment (start 95.779242 130.069242) (end 95.779242 130.121989) (width 0.25) (layer F.Cu) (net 16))
 (via (at 95.779242 130.121989) (size 0.8) (drill 0.4) (layers F.Cu B.Cu) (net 16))
 (segment (start 95.504 129.794) (end 95.779242 130.069242) (width 0.25) (layer F.Cu) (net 16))
 (segment (start 95.379243 130.521988) (end 95.779242 130.121989) (width 0.25) (layer B.Cu) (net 16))
 (segment (start 109.211 123.698) (end 109.474 123.435) (width 0.25) (layer F.Cu) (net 17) (status 30))
 (segment (start 106.172 123.698) (end 109.211 123.698) (width 0.25) (layer F.Cu) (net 17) (status 30))
 (segment (start 114.93359 126.238) (end 116.078 126.238) (width 0.25) (layer F.Cu) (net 18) (status 20))
 (segment (start 113.557218 124.861628) (end 114.93359 126.238) (width 0.25) (layer F.Cu) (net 18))
 (segment (start 109.474 125.485) (end 110.097372 124.861628) (width 0.25) (layer F.Cu) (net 18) (status 10))
 (segment (start 110.097372 124.861628) (end 113.557218 124.861628) (width 0.25) (layer F.Cu) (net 18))
 (segment (start 105.04699 128.92299) (end 106.172 130.048) (width 0.25) (layer F.Cu) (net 19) (status 20))
 (segment (start 103.372 123.698) (end 103.372 124.32841) (width 0.25) (layer F.Cu) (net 19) (status 30))
 (segment (start 105.04699 126.0034) (end 105.04699 128.92299) (width 0.25) (layer F.Cu) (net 19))
 (segment (start 103.372 124.32841) (end 105.04699 126.0034) (width 0.25) (layer F.Cu) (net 19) (status 10))
 (segment (start 105.04699 128.92299) (end 101.004012 128.92299) (width 0.25) (layer F.Cu) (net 19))
 (segment (start 97.536 132.391002) (end 97.536 137.367823) (width 0.25) (layer F.Cu) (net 19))
 (segment (start 101.004012 128.92299) (end 97.536 132.391002) (width 0.25) (layer F.Cu) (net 19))
 (segment (start 97.536 137.367823) (end 93.171823 141.732) (width 0.25) (layer F.Cu) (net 19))
 (segment (start 80.626 141.732) (end 78.994 140.1) (width 0.25) (layer F.Cu) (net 19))
 (segment (start 93.171823 141.732) (end 80.626 141.732) (width 0.25) (layer F.Cu) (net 19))
 (segment (start 78.994 140.1) (end 78.994 139.7) (width 0.25) (layer F.Cu) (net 19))
 (via (at 97.028008 130.048) (size 0.8) (drill 0.4) (layers F.Cu B.Cu) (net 21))
 (segment (start 116.332 127.897422) (end 116.332 129.803) (width 0.25) (layer F.Cu) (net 21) (status 20))
 (segment (start 113.278 123.946) (end 114.44499 125.11299) (width 0.25) (layer F.Cu) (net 21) (status 10))
 (segment (start 113.278 123.698) (end 113.278 123.946) (width 0.25) (layer F.Cu) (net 21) (status 30))
 (segment (start 114.44499 125.11299) (end 116.866412 125.11299) (width 0.25) (layer F.Cu) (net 21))
 (segment (start 116.866412 125.11299) (end 117.20301 125.449588) (width 0.25) (layer F.Cu) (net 21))
 (segment (start 116.332 129.803) (end 116.087 130.048) (width 0.25) (layer F.Cu) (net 21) (status 30))
 (segment (start 117.20301 125.449588) (end 117.20301 127.026412) (width 0.25) (layer F.Cu) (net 21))
 (segment (start 117.20301 127.026412) (end 116.332 127.897422) (width 0.25) (layer F.Cu) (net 21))
 (segment (start 98.189999 128.886009) (end 97.028008 130.048) (width 0.25) (layer F.Cu) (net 21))
 (segment (start 98.189999 125.076001) (end 98.189999 128.886009) (width 0.25) (layer F.Cu) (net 21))
 (segment (start 102.362 120.904) (end 98.189999 125.076001) (width 0.25) (layer F.Cu) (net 21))
 (segment (start 113.278 123.698) (end 110.484 120.904) (width 0.25) (layer F.Cu) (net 21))
 (segment (start 110.484 120.904) (end 102.362 120.904) (width 0.25) (layer F.Cu) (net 21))
 (segment (start 97.028008 131.825996) (end 97.028012 131.826) (width 0.25) (layer B.Cu) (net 21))
 (segment (start 85.255989 141.281989) (end 92.985423 141.281989) (width 0.25) (layer F.Cu) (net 21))
 (segment (start 97.028008 130.048) (end 97.028008 131.825996) (width 0.25) (layer B.Cu) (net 21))
 (segment (start 97.028012 132.391685) (end 97.028012 131.826) (width 0.25) (layer F.Cu) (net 21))
 (segment (start 92.985423 141.281989) (end 97.028012 137.2394) (width 0.25) (layer F.Cu) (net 21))
 (segment (start 97.028012 137.2394) (end 97.028012 132.391685) (width 0.25) (layer F.Cu) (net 21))
 (segment (start 84.074 139.7) (end 84.074 140.1) (width 0.25) (layer F.Cu) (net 21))
 (segment (start 84.074 140.1) (end 85.255989 141.281989) (width 0.25) (layer F.Cu) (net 21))
 (via (at 97.028012 131.826) (size 0.8) (drill 0.4) (layers F.Cu B.Cu) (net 21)))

